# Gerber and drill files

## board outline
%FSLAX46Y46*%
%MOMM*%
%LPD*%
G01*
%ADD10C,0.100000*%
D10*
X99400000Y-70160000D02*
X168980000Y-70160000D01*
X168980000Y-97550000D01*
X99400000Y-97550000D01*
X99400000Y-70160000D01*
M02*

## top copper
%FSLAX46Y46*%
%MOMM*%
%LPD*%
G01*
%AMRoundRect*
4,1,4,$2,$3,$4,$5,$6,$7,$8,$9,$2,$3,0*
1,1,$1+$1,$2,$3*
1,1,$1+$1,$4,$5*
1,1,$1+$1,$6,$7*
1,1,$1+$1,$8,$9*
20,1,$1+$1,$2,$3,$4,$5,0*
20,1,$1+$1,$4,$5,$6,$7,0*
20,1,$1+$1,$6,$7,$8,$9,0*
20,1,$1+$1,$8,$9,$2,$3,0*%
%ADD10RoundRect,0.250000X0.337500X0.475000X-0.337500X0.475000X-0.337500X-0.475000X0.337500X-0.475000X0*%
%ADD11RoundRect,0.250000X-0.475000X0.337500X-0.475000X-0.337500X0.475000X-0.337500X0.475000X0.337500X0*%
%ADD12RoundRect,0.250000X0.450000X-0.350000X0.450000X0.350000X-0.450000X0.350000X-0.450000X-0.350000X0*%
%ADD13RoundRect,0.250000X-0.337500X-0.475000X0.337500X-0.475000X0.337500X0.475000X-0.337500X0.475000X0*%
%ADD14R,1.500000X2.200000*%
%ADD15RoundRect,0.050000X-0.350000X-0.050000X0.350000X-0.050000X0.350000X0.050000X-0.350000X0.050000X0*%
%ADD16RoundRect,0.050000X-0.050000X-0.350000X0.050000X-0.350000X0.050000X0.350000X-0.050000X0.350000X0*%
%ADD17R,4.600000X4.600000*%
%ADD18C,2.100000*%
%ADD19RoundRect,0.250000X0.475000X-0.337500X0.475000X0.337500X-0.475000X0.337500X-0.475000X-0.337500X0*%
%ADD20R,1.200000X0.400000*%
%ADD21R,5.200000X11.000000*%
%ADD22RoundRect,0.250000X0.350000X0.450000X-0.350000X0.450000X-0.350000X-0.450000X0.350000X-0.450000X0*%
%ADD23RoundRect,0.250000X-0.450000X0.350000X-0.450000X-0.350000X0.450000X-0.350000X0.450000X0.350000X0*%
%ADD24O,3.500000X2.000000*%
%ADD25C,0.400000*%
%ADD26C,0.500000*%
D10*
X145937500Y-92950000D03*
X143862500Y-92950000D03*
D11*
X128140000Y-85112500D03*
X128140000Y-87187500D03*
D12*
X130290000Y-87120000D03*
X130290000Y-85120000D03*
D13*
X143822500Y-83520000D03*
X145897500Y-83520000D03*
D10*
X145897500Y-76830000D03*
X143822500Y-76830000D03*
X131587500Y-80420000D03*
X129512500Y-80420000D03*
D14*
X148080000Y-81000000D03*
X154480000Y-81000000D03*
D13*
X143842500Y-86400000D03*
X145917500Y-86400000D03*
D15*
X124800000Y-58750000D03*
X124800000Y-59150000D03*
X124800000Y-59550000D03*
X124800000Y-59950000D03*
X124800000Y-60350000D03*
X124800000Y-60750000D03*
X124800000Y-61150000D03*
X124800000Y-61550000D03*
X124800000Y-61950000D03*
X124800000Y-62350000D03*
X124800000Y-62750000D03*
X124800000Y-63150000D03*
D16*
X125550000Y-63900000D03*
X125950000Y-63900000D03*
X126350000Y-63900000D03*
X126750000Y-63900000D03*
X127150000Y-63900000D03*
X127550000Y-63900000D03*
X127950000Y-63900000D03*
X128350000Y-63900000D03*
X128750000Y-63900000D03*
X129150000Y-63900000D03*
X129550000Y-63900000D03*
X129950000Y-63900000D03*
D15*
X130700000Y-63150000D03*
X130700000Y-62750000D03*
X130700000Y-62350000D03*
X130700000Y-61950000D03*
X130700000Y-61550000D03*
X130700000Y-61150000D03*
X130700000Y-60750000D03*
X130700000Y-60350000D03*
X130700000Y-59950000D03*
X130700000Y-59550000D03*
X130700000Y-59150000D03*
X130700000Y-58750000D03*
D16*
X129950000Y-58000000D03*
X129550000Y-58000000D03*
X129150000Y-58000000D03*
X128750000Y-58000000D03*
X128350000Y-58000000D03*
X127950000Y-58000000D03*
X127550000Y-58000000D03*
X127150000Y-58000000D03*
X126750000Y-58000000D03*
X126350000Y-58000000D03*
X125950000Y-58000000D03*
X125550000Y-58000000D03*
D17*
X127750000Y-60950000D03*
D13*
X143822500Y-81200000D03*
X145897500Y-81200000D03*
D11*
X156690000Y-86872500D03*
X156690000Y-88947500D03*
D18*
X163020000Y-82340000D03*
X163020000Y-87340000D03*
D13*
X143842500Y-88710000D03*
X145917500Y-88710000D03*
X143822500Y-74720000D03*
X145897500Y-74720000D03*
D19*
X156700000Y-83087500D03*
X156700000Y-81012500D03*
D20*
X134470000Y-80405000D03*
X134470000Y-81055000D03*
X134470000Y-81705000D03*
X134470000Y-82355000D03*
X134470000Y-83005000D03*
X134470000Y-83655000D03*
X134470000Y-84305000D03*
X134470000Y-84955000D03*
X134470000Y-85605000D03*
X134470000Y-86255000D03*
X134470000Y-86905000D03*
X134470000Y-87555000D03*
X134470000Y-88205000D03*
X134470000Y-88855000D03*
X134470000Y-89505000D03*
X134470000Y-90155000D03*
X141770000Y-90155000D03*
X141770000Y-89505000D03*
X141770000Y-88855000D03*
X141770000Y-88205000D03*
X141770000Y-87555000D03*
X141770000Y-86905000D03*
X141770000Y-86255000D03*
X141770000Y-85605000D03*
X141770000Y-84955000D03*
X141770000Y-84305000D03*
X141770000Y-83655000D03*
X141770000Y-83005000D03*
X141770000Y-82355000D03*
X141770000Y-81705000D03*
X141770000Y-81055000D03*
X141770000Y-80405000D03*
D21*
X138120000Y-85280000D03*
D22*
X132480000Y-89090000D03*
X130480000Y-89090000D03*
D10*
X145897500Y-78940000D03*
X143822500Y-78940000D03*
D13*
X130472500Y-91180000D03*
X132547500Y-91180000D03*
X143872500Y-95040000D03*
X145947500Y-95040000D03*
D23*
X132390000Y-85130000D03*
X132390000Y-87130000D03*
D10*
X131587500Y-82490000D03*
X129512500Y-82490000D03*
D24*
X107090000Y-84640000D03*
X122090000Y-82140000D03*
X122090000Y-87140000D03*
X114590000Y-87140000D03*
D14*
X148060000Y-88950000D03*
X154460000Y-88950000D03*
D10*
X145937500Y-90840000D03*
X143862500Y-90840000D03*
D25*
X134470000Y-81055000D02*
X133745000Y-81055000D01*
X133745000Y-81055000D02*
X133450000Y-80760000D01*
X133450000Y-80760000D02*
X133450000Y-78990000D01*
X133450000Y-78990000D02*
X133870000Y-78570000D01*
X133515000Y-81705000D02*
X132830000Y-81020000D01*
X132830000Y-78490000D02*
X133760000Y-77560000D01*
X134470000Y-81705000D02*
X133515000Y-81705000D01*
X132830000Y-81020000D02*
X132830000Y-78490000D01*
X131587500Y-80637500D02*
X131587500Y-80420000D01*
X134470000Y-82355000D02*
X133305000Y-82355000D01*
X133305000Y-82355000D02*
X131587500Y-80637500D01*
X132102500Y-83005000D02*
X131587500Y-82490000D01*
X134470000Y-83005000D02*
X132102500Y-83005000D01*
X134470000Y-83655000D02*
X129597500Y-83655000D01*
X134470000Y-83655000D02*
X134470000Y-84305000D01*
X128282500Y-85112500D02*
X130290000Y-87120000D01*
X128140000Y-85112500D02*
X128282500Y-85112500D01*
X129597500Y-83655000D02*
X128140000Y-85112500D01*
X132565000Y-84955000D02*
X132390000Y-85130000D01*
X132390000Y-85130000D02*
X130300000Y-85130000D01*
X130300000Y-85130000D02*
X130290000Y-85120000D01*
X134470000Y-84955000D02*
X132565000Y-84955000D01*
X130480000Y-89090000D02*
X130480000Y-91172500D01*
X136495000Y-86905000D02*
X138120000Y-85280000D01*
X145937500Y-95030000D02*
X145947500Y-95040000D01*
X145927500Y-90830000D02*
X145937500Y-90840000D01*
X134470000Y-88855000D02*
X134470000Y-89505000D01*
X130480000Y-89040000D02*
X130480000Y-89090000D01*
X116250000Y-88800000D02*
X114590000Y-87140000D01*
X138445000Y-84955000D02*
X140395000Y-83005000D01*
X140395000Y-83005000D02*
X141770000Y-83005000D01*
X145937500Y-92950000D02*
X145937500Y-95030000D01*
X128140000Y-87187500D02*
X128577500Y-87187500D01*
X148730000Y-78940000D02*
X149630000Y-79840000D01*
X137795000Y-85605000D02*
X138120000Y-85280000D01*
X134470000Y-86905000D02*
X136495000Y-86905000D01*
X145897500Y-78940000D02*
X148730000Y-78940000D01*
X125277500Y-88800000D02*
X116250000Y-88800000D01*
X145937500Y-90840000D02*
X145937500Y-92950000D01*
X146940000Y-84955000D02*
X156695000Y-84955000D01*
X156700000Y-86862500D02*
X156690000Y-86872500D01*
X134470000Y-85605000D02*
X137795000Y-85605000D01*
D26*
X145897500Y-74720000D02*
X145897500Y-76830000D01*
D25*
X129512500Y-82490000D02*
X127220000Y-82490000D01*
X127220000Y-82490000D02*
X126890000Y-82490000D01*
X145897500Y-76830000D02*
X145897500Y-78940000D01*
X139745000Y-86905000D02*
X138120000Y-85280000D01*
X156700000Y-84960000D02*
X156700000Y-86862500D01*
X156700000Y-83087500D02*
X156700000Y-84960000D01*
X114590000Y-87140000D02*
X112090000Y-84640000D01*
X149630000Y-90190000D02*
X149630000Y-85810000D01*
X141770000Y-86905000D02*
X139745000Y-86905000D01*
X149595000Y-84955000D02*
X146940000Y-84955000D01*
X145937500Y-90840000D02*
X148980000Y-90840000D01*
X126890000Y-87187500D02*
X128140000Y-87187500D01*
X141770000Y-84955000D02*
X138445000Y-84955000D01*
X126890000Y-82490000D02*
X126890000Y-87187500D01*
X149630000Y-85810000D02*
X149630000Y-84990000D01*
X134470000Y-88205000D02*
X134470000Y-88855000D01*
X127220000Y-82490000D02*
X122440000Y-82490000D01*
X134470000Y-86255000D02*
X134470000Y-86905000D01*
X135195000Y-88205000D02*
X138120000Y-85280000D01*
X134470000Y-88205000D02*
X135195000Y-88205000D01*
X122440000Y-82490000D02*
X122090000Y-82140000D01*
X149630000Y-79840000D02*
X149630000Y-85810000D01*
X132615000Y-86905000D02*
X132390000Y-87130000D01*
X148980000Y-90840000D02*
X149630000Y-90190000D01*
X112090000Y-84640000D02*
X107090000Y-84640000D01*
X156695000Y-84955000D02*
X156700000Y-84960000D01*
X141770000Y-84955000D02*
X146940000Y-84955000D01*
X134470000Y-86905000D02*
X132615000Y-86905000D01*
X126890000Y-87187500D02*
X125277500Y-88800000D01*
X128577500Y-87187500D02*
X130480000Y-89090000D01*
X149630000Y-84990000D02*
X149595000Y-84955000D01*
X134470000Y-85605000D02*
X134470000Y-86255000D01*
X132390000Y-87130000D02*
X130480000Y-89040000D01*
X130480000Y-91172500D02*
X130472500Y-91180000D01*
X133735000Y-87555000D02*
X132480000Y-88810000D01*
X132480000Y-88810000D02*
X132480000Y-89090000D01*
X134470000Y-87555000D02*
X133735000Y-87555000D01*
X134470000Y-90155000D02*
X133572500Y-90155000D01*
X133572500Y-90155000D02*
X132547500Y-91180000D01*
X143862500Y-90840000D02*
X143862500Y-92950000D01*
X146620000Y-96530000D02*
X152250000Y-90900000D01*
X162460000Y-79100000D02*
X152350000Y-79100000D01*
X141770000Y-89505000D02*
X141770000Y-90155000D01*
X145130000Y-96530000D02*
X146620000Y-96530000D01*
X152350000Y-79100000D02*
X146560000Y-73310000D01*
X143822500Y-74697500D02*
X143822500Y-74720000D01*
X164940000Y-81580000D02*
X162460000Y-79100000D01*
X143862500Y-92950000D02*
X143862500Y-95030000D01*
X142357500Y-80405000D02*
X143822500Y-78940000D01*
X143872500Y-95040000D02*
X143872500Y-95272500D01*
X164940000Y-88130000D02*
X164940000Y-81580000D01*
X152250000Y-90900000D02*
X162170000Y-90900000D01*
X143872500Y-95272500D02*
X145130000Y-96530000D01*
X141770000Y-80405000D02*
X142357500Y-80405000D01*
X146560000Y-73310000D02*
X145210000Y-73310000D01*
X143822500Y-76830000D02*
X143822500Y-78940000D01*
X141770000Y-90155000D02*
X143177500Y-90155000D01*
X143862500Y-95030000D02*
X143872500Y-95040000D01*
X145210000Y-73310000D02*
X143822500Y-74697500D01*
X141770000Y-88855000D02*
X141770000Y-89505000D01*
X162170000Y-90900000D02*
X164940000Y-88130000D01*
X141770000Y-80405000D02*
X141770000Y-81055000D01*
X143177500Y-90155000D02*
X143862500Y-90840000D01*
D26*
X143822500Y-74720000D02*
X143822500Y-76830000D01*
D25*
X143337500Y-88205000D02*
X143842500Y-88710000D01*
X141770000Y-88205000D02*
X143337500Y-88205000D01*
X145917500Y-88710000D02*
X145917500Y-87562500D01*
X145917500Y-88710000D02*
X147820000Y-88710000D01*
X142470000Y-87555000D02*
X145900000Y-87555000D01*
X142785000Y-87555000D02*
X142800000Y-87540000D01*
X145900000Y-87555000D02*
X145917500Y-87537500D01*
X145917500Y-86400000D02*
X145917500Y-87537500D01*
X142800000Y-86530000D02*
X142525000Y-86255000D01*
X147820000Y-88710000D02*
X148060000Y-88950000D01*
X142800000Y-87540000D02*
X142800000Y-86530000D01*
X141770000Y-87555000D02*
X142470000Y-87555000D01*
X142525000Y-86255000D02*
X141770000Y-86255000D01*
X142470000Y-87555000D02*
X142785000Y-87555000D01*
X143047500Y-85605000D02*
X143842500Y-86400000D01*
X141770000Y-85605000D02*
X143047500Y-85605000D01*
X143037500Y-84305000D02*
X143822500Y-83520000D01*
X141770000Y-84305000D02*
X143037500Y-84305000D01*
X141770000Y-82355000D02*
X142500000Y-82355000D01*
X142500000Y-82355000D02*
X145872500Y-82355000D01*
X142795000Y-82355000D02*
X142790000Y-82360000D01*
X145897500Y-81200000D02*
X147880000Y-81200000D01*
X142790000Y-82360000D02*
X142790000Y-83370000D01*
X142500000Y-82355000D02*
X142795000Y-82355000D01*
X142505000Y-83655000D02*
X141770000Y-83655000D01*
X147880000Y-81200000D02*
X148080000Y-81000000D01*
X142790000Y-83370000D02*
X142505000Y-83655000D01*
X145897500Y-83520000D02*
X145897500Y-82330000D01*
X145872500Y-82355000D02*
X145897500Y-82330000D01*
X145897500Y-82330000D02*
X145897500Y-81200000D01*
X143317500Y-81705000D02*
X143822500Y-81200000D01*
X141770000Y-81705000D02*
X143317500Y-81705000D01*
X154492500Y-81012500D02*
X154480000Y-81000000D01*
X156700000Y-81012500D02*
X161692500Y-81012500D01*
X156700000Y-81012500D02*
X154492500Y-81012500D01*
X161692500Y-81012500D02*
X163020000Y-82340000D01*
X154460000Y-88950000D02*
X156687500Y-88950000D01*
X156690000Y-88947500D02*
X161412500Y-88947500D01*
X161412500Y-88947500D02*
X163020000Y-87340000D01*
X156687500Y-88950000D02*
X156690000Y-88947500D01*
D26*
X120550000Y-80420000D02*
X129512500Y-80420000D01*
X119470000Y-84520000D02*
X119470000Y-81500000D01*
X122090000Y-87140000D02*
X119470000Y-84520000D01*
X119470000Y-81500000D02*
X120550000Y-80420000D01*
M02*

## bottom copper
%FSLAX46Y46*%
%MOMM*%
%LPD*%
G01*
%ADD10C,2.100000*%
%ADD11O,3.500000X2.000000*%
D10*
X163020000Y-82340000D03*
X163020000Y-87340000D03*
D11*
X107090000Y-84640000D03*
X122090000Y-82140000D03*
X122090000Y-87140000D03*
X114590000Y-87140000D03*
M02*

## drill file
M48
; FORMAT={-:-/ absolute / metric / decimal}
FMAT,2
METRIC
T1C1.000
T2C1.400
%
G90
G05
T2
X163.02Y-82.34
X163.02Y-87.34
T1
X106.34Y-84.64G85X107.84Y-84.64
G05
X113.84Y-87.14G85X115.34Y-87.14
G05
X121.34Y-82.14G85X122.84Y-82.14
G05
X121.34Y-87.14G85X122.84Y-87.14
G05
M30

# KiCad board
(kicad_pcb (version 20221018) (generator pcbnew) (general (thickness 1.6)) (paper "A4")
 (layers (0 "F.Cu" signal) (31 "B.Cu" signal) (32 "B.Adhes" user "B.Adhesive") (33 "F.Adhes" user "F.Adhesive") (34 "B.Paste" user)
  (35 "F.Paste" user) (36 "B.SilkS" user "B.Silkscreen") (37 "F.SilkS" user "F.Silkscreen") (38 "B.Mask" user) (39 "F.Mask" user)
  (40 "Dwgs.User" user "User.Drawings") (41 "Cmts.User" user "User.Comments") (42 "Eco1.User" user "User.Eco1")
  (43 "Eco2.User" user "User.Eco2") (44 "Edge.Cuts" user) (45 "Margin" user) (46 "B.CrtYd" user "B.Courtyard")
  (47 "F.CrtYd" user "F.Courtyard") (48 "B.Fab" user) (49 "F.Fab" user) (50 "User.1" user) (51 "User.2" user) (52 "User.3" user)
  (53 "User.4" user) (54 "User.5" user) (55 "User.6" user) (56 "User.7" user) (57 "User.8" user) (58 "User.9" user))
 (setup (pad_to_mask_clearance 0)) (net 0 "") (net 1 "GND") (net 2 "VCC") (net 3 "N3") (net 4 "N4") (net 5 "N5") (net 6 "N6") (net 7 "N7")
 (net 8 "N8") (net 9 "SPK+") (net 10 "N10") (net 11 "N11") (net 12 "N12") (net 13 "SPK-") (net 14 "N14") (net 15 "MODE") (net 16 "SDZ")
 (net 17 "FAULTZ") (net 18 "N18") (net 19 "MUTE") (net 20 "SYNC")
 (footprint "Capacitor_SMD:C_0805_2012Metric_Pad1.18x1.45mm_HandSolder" (layer "F.Cu") (at 144.9 92.95 180)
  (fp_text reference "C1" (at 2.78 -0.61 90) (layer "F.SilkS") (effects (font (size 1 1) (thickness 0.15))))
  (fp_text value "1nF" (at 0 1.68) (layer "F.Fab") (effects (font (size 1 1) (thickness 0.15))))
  (pad "1" smd roundrect (at -1.0375 0 180) (size 1.175 1.45) (layers "F.Cu" "F.Paste" "F.Mask") (roundrect_rratio 0.212766) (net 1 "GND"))
  (pad "2" smd roundrect (at 1.0375 0 180) (size 1.175 1.45) (layers "F.Cu" "F.Paste" "F.Mask") (roundrect_rratio 0.212766) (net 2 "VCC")))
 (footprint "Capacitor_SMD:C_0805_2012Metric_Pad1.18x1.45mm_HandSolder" (layer "F.Cu") (at 128.14 86.15 -90)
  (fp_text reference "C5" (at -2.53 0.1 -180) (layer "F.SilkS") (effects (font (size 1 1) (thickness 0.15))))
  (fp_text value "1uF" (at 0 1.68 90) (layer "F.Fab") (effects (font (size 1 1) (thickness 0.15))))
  (pad "1" smd roundrect (at -1.0375 0 270) (size 1.175 1.45) (layers "F.Cu" "F.Paste" "F.Mask") (roundrect_rratio 0.212766) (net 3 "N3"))
  (pad "2" smd roundrect (at 1.0375 0 270) (size 1.175 1.45) (layers "F.Cu" "F.Paste" "F.Mask") (roundrect_rratio 0.212766) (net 1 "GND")))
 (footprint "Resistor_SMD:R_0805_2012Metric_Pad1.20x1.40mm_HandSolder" (layer "F.Cu") (at 130.29 86.12 90)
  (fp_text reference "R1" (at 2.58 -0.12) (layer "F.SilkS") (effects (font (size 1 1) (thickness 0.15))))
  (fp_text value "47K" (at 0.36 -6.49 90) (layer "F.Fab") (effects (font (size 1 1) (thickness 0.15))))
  (pad "1" smd roundrect (at -1 0 90) (size 1.2 1.4) (layers "F.Cu" "F.Paste" "F.Mask") (roundrect_rratio 0.208333) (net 3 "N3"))
  (pad "2" smd roundrect (at 1 0 90) (size 1.2 1.4) (layers "F.Cu" "F.Paste" "F.Mask") (roundrect_rratio 0.208333) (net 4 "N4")))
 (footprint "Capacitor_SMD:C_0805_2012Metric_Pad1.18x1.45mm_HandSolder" (layer "F.Cu") (at 144.86 83.52)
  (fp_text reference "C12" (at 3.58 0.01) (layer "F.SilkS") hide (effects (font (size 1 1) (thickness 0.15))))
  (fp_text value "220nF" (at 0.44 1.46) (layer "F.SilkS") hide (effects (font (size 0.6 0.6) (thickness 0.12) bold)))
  (pad "1" smd roundrect (at -1.0375 0) (size 1.175 1.45) (layers "F.Cu" "F.Paste" "F.Mask") (roundrect_rratio 0.212766) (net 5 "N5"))
  (pad "2" smd roundrect (at 1.0375 0) (size 1.175 1.45) (layers "F.Cu" "F.Paste" "F.Mask") (roundrect_rratio 0.212766) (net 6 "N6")))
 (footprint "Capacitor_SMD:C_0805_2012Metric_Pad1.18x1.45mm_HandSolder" (layer "F.Cu") (at 144.86 76.83 180)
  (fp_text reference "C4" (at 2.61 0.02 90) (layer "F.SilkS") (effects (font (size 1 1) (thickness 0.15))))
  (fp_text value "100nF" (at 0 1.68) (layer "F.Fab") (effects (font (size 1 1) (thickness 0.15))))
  (pad "1" smd roundrect (at -1.0375 0 180) (size 1.175 1.45) (layers "F.Cu" "F.Paste" "F.Mask") (roundrect_rratio 0.212766) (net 1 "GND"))
  (pad "2" smd roundrect (at 1.0375 0 180) (size 1.175 1.45) (layers "F.Cu" "F.Paste" "F.Mask") (roundrect_rratio 0.212766) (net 2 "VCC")))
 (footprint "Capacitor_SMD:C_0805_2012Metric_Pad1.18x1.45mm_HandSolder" (layer "F.Cu") (at 130.55 80.42 180)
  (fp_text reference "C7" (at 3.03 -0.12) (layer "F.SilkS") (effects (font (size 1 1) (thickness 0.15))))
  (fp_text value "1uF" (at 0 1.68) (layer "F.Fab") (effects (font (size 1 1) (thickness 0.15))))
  (pad "1" smd roundrect (at -1.0375 0 180) (size 1.175 1.45) (layers "F.Cu" "F.Paste" "F.Mask") (roundrect_rratio 0.212766) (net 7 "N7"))
  (pad "2" smd roundrect (at 1.0375 0 180) (size 1.175 1.45) (layers "F.Cu" "F.Paste" "F.Mask") (roundrect_rratio 0.212766) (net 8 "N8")))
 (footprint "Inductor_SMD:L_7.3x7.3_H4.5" (layer "F.Cu") (at 151.28 81)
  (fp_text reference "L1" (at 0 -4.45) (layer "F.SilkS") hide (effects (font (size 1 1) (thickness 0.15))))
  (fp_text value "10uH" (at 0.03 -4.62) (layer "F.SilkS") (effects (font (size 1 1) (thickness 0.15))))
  (pad "1" smd rect (at -3.2 0) (size 1.5 2.2) (layers "F.Cu" "F.Paste" "F.Mask") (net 6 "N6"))
  (pad "2" smd rect (at 3.2 0) (size 1.5 2.2) (layers "F.Cu" "F.Paste" "F.Mask") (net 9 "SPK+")))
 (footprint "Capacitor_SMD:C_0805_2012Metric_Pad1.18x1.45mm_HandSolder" (layer "F.Cu") (at 144.88 86.4)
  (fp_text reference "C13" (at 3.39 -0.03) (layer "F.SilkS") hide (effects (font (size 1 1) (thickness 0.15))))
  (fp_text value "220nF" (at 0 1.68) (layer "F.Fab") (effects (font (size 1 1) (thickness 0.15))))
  (pad "1" smd roundrect (at -1.0375 0) (size 1.175 1.45) (layers "F.Cu" "F.Paste" "F.Mask") (roundrect_rratio 0.212766) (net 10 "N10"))
  (pad "2" smd roundrect (at 1.0375 0) (size 1.175 1.45) (layers "F.Cu" "F.Paste" "F.Mask") (roundrect_rratio 0.212766) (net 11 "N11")))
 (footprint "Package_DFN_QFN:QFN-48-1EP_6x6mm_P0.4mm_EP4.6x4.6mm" (layer "F.Cu") (at 127.75 60.95)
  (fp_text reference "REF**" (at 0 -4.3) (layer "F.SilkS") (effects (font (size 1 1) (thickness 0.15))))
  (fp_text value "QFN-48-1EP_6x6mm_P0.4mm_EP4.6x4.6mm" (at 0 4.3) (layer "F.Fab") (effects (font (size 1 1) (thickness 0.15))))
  (pad "" smd roundrect (at -1.53 -1.53) (size 1.24 1.24) (layers "F.Paste") (roundrect_rratio 0.201613))
  (pad "" smd roundrect (at -1.53 0) (size 1.24 1.24) (layers "F.Paste") (roundrect_rratio 0.201613))
  (pad "" smd roundrect (at -1.53 1.53) (size 1.24 1.24) (layers "F.Paste") (roundrect_rratio 0.201613))
  (pad "" smd roundrect (at 0 -1.53) (size 1.24 1.24) (layers "F.Paste") (roundrect_rratio 0.201613))
  (pad "" smd roundrect (at 0 0) (size 1.24 1.24) (layers "F.Paste") (roundrect_rratio 0.201613))
  (pad "" smd roundrect (at 0 1.53) (size 1.24 1.24) (layers "F.Paste") (roundrect_rratio 0.201613))
  (pad "" smd roundrect (at 1.53 -1.53) (size 1.24 1.24) (layers "F.Paste") (roundrect_rratio 0.201613))
  (pad "" smd roundrect (at 1.53 0) (size 1.24 1.24) (layers "F.Paste") (roundrect_rratio 0.201613))
  (pad "" smd roundrect (at 1.53 1.53) (size 1.24 1.24) (layers "F.Paste") (roundrect_rratio 0.201613))
  (pad "1" smd roundrect (at -2.95 -2.2) (size 0.8 0.2) (layers "F.Cu" "F.Paste" "F.Mask") (roundrect_rratio 0.25))
  (pad "2" smd roundrect (at -2.95 -1.8) (size 0.8 0.2) (layers "F.Cu" "F.Paste" "F.Mask") (roundrect_rratio 0.25))
  (pad "3" smd roundrect (at -2.95 -1.4) (size 0.8 0.2) (layers "F.Cu" "F.Paste" "F.Mask") (roundrect_rratio 0.25))
  (pad "4" smd roundrect (at -2.95 -1) (size 0.8 0.2) (layers "F.Cu" "F.Paste" "F.Mask") (roundrect_rratio 0.25))
  (pad "5" smd roundrect (at -2.95 -0.6) (size 0.8 0.2) (layers "F.Cu" "F.Paste" "F.Mask") (roundrect_rratio 0.25))
  (pad "6" smd roundrect (at -2.95 -0.2) (size 0.8 0.2) (layers "F.Cu" "F.Paste" "F.Mask") (roundrect_rratio 0.25))
  (pad "7" smd roundrect (at -2.95 0.2) (size 0.8 0.2) (layers "F.Cu" "F.Paste" "F.Mask") (roundrect_rratio 0.25))
  (pad "8" smd roundrect (at -2.95 0.6) (size 0.8 0.2) (layers "F.Cu" "F.Paste" "F.Mask") (roundrect_rratio 0.25))
  (pad "9" smd roundrect (at -2.95 1) (size 0.8 0.2) (layers "F.Cu" "F.Paste" "F.Mask") (roundrect_rratio 0.25))
  (pad "10" smd roundrect (at -2.95 1.4) (size 0.8 0.2) (layers "F.Cu" "F.Paste" "F.Mask") (roundrect_rratio 0.25))
  (pad "11" smd roundrect (at -2.95 1.8) (size 0.8 0.2) (layers "F.Cu" "F.Paste" "F.Mask") (roundrect_rratio 0.25))
  (pad "12" smd roundrect (at -2.95 2.2) (size 0.8 0.2) (layers "F.Cu" "F.Paste" "F.Mask") (roundrect_rratio 0.25))
  (pad "13" smd roundrect (at -2.2 2.95) (size 0.2 0.8) (layers "F.Cu" "F.Paste" "F.Mask") (roundrect_rratio 0.25))
  (pad "14" smd roundrect (at -1.8 2.95) (size 0.2 0.8) (layers "F.Cu" "F.Paste" "F.Mask") (roundrect_rratio 0.25))
  (pad "15" smd roundrect (at -1.4 2.95) (size 0.2 0.8) (layers "F.Cu" "F.Paste" "F.Mask") (roundrect_rratio 0.25))
  (pad "16" smd roundrect (at -1 2.95) (size 0.2 0.8) (layers "F.Cu" "F.Paste" "F.Mask") (roundrect_rratio 0.25))
  (pad "17" smd roundrect (at -0.6 2.95) (size 0.2 0.8) (layers "F.Cu" "F.Paste" "F.Mask") (roundrect_rratio 0.25))
  (pad "18" smd roundrect (at -0.2 2.95) (size 0.2 0.8) (layers "F.Cu" "F.Paste" "F.Mask") (roundrect_rratio 0.25))
  (pad "19" smd roundrect (at 0.2 2.95) (size 0.2 0.8) (layers "F.Cu" "F.Paste" "F.Mask") (roundrect_rratio 0.25))
  (pad "20" smd roundrect (at 0.6 2.95) (size 0.2 0.8) (layers "F.Cu" "F.Paste" "F.Mask") (roundrect_rratio 0.25))
  (pad "21" smd roundrect (at 1 2.95) (size 0.2 0.8) (layers "F.Cu" "F.Paste" "F.Mask") (roundrect_rratio 0.25))
  (pad "22" smd roundrect (at 1.4 2.95) (size 0.2 0.8) (layers "F.Cu" "F.Paste" "F.Mask") (roundrect_rratio 0.25))
  (pad "23" smd roundrect (at 1.8 2.95) (size 0.2 0.8) (layers "F.Cu" "F.Paste" "F.Mask") (roundrect_rratio 0.25))
  (pad "24" smd roundrect (at 2.2 2.95) (size 0.2 0.8) (layers "F.Cu" "F.Paste" "F.Mask") (roundrect_rratio 0.25))
  (pad "25" smd roundrect (at 2.95 2.2) (size 0.8 0.2) (layers "F.Cu" "F.Paste" "F.Mask") (roundrect_rratio 0.25))
  (pad "26" smd roundrect (at 2.95 1.8) (size 0.8 0.2) (layers "F.Cu" "F.Paste" "F.Mask") (roundrect_rratio 0.25))
  (pad "27" smd roundrect (at 2.95 1.4) (size 0.8 0.2) (layers "F.Cu" "F.Paste" "F.Mask") (roundrect_rratio 0.25))
  (pad "28" smd roundrect (at 2.95 1) (size 0.8 0.2) (layers "F.Cu" "F.Paste" "F.Mask") (roundrect_rratio 0.25))
  (pad "29" smd roundrect (at 2.95 0.6) (size 0.8 0.2) (layers "F.Cu" "F.Paste" "F.Mask") (roundrect_rratio 0.25))
  (pad "30" smd roundrect (at 2.95 0.2) (size 0.8 0.2) (layers "F.Cu" "F.Paste" "F.Mask") (roundrect_rratio 0.25))
  (pad "31" smd roundrect (at 2.95 -0.2) (size 0.8 0.2) (layers "F.Cu" "F.Paste" "F.Mask") (roundrect_rratio 0.25))
  (pad "32" smd roundrect (at 2.95 -0.6) (size 0.8 0.2) (layers "F.Cu" "F.Paste" "F.Mask") (roundrect_rratio 0.25))
  (pad "33" smd roundrect (at 2.95 -1) (size 0.8 0.2) (layers "F.Cu" "F.Paste" "F.Mask") (roundrect_rratio 0.25))
  (pad "34" smd roundrect (at 2.95 -1.4) (size 0.8 0.2) (layers "F.Cu" "F.Paste" "F.Mask") (roundrect_rratio 0.25))
  (pad "35" smd roundrect (at 2.95 -1.8) (size 0.8 0.2) (layers "F.Cu" "F.Paste" "F.Mask") (roundrect_rratio 0.25))
  (pad "36" smd roundrect (at 2.95 -2.2) (size 0.8 0.2) (layers "F.Cu" "F.Paste" "F.Mask") (roundrect_rratio 0.25))
  (pad "37" smd roundrect (at 2.2 -2.95) (size 0.2 0.8) (layers "F.Cu" "F.Paste" "F.Mask") (roundrect_rratio 0.25))
  (pad "38" smd roundrect (at 1.8 -2.95) (size 0.2 0.8) (layers "F.Cu" "F.Paste" "F.Mask") (roundrect_rratio 0.25))
  (pad "39" smd roundrect (at 1.4 -2.95) (size 0.2 0.8) (layers "F.Cu" "F.Paste" "F.Mask") (roundrect_rratio 0.25))
  (pad "40" smd roundrect (at 1 -2.95) (size 0.2 0.8) (layers "F.Cu" "F.Paste" "F.Mask") (roundrect_rratio 0.25))
  (pad "41" smd roundrect (at 0.6 -2.95) (size 0.2 0.8) (layers "F.Cu" "F.Paste" "F.Mask") (roundrect_rratio 0.25))
  (pad "42" smd roundrect (at 0.2 -2.95) (size 0.2 0.8) (layers "F.Cu" "F.Paste" "F.Mask") (roundrect_rratio 0.25))
  (pad "43" smd roundrect (at -0.2 -2.95) (size 0.2 0.8) (layers "F.Cu" "F.Paste" "F.Mask") (roundrect_rratio 0.25))
  (pad "44" smd roundrect (at -0.6 -2.95) (size 0.2 0.8) (layers "F.Cu" "F.Paste" "F.Mask") (roundrect_rratio 0.25))
  (pad "45" smd roundrect (at -1 -2.95) (size 0.2 0.8) (layers "F.Cu" "F.Paste" "F.Mask") (roundrect_rratio 0.25))
  (pad "46" smd roundrect (at -1.4 -2.95) (size 0.2 0.8) (layers "F.Cu" "F.Paste" "F.Mask") (roundrect_rratio 0.25))
  (pad "47" smd roundrect (at -1.8 -2.95) (size 0.2 0.8) (layers "F.Cu" "F.Paste" "F.Mask") (roundrect_rratio 0.25))
  (pad "48" smd roundrect (at -2.2 -2.95) (size 0.2 0.8) (layers "F.Cu" "F.Paste" "F.Mask") (roundrect_rratio 0.25))
  (pad "49" smd rect (at 0 0) (size 4.6 4.6) (layers "F.Cu" "F.Mask")))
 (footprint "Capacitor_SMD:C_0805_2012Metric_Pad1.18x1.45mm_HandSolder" (layer "F.Cu") (at 144.86 81.2)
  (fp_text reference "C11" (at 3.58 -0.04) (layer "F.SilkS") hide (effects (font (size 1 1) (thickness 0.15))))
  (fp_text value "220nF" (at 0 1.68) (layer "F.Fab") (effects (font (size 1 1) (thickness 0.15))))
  (pad "1" smd roundrect (at -1.0375 0) (size 1.175 1.45) (layers "F.Cu" "F.Paste" "F.Mask") (roundrect_rratio 0.212766) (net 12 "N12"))
  (pad "2" smd roundrect (at 1.0375 0) (size 1.175 1.45) (layers "F.Cu" "F.Paste" "F.Mask") (roundrect_rratio 0.212766) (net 6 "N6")))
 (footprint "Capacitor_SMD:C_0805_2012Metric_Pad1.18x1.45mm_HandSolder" (layer "F.Cu") (at 156.69 87.91 -90)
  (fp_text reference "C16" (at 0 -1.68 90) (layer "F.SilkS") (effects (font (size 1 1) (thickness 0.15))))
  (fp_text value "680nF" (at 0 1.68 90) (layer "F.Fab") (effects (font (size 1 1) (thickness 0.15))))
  (pad "1" smd roundrect (at -1.0375 0 270) (size 1.175 1.45) (layers "F.Cu" "F.Paste" "F.Mask") (roundrect_rratio 0.212766) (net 1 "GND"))
  (pad "2" smd roundrect (at 1.0375 0 270) (size 1.175 1.45) (layers "F.Cu" "F.Paste" "F.Mask") (roundrect_rratio 0.212766) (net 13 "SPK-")))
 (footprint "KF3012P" (layer "F.Cu") (at 163.02 82.34 -90)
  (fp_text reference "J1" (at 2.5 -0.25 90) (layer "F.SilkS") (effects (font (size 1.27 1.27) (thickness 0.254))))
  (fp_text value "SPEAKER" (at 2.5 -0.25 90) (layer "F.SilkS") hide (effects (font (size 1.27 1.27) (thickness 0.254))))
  (pad "1" thru_hole circle (at 0 0 270) (size 2.1 2.1) (drill 1.4) (layers "*.Cu" "*.Mask") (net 9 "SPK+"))
  (pad "2" thru_hole circle (at 5 0 270) (size 2.1 2.1) (drill 1.4) (layers "*.Cu" "*.Mask") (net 13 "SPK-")))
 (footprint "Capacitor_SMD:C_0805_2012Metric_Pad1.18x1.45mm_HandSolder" (layer "F.Cu") (at 144.88 88.71)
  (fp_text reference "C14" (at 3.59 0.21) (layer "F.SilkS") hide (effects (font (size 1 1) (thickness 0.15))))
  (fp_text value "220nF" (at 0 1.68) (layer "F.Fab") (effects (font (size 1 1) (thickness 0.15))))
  (pad "1" smd roundrect (at -1.0375 0) (size 1.175 1.45) (layers "F.Cu" "F.Paste" "F.Mask") (roundrect_rratio 0.212766) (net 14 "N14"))
  (pad "2" smd roundrect (at 1.0375 0) (size 1.175 1.45) (layers "F.Cu" "F.Paste" "F.Mask") (roundrect_rratio 0.212766) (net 11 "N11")))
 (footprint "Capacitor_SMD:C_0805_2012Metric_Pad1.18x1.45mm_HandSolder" (layer "F.Cu") (at 144.86 74.72)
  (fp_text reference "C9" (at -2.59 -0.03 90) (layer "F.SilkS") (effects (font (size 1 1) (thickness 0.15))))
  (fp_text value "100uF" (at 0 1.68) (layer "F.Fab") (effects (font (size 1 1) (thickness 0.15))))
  (pad "1" smd roundrect (at -1.0375 0) (size 1.175 1.45) (layers "F.Cu" "F.Paste" "F.Mask") (roundrect_rratio 0.212766) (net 2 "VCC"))
  (pad "2" smd roundrect (at 1.0375 0) (size 1.175 1.45) (layers "F.Cu" "F.Paste" "F.Mask") (roundrect_rratio 0.212766) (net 1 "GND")))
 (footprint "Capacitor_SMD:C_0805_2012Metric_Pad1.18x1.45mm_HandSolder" (layer "F.Cu") (at 156.7 82.05 90)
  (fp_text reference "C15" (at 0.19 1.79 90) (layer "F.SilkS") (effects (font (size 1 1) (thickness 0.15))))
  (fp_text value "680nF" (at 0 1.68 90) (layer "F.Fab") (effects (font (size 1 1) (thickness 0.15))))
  (pad "1" smd roundrect (at -1.0375 0 90) (size 1.175 1.45) (layers "F.Cu" "F.Paste" "F.Mask") (roundrect_rratio 0.212766) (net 1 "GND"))
  (pad "2" smd roundrect (at 1.0375 0 90) (size 1.175 1.45) (layers "F.Cu" "F.Paste" "F.Mask") (roundrect_rratio 0.212766) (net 9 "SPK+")))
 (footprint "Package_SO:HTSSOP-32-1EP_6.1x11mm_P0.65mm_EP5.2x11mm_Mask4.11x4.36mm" (layer "F.Cu") (at 138.12 85.28)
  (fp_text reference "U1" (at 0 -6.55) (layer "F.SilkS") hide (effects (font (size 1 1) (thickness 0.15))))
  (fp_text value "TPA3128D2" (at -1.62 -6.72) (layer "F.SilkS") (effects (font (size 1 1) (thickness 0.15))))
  (pad "" smd rect (at -1.37 -1.46) (size 1.07 1.16) (layers "F.Paste"))
  (pad "" smd rect (at -1.37 0) (size 1.07 1.16) (layers "F.Paste"))
  (pad "" smd rect (at -1.37 1.46) (size 1.07 1.16) (layers "F.Paste"))
  (pad "" smd rect (at 0 -1.46) (size 1.07 1.16) (layers "F.Paste"))
  (pad "" smd rect (at 0 0) (size 1.07 1.16) (layers "F.Paste"))
  (pad "" smd rect (at 0 0) (size 4.11 4.36) (layers "F.Mask"))
  (pad "" smd rect (at 0 1.46) (size 1.07 1.16) (layers "F.Paste"))
  (pad "" smd rect (at 1.37 -1.46) (size 1.07 1.16) (layers "F.Paste"))
  (pad "" smd rect (at 1.37 0) (size 1.07 1.16) (layers "F.Paste"))
  (pad "" smd rect (at 1.37 1.46) (size 1.07 1.16) (layers "F.Paste"))
  (pad "1" smd rect (at -3.65 -4.875) (size 1.2 0.4) (layers "F.Cu" "F.Paste" "F.Mask") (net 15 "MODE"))
  (pad "2" smd rect (at -3.65 -4.225) (size 1.2 0.4) (layers "F.Cu" "F.Paste" "F.Mask") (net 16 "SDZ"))
  (pad "3" smd rect (at -3.65 -3.575) (size 1.2 0.4) (layers "F.Cu" "F.Paste" "F.Mask") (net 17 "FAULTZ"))
  (pad "4" smd rect (at -3.65 -2.925) (size 1.2 0.4) (layers "F.Cu" "F.Paste" "F.Mask") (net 7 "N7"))
  (pad "5" smd rect (at -3.65 -2.275) (size 1.2 0.4) (layers "F.Cu" "F.Paste" "F.Mask") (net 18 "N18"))
  (pad "6" smd rect (at -3.65 -1.625) (size 1.2 0.4) (layers "F.Cu" "F.Paste" "F.Mask") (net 3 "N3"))
  (pad "7" smd rect (at -3.65 -0.975) (size 1.2 0.4) (layers "F.Cu" "F.Paste" "F.Mask") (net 3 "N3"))
  (pad "8" smd rect (at -3.65 -0.325) (size 1.2 0.4) (layers "F.Cu" "F.Paste" "F.Mask") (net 4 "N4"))
  (pad "9" smd rect (at -3.65 0.325) (size 1.2 0.4) (layers "F.Cu" "F.Paste" "F.Mask") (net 1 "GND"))
  (pad "10" smd rect (at -3.65 0.975) (size 1.2 0.4) (layers "F.Cu" "F.Paste" "F.Mask") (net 1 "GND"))
  (pad "11" smd rect (at -3.65 1.625) (size 1.2 0.4) (layers "F.Cu" "F.Paste" "F.Mask") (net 1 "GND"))
  (pad "12" smd rect (at -3.65 2.275) (size 1.2 0.4) (layers "F.Cu" "F.Paste" "F.Mask") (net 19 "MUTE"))
  (pad "13" smd rect (at -3.65 2.925) (size 1.2 0.4) (layers "F.Cu" "F.Paste" "F.Mask") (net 1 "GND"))
  (pad "14" smd rect (at -3.65 3.575) (size 1.2 0.4) (layers "F.Cu" "F.Paste" "F.Mask") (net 1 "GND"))
  (pad "15" smd rect (at -3.65 4.225) (size 1.2 0.4) (layers "F.Cu" "F.Paste" "F.Mask") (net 1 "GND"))
  (pad "16" smd rect (at -3.65 4.875) (size 1.2 0.4) (layers "F.Cu" "F.Paste" "F.Mask") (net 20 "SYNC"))
  (pad "17" smd rect (at 3.65 4.875) (size 1.2 0.4) (layers "F.Cu" "F.Paste" "F.Mask") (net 2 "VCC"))
  (pad "18" smd rect (at 3.65 4.225) (size 1.2 0.4) (layers "F.Cu" "F.Paste" "F.Mask") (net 2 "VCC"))
  (pad "19" smd rect (at 3.65 3.575) (size 1.2 0.4) (layers "F.Cu" "F.Paste" "F.Mask") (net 2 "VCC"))
  (pad "20" smd rect (at 3.65 2.925) (size 1.2 0.4) (layers "F.Cu" "F.Paste" "F.Mask") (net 14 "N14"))
  (pad "21" smd rect (at 3.65 2.275) (size 1.2 0.4) (layers "F.Cu" "F.Paste" "F.Mask") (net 11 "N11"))
  (pad "22" smd rect (at 3.65 1.625) (size 1.2 0.4) (layers "F.Cu" "F.Paste" "F.Mask") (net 1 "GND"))
  (pad "23" smd rect (at 3.65 0.975) (size 1.2 0.4) (layers "F.Cu" "F.Paste" "F.Mask") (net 11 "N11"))
  (pad "24" smd rect (at 3.65 0.325) (size 1.2 0.4) (layers "F.Cu" "F.Paste" "F.Mask") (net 10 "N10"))
  (pad "25" smd rect (at 3.65 -0.325) (size 1.2 0.4) (layers "F.Cu" "F.Paste" "F.Mask") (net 1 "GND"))
  (pad "26" smd rect (at 3.65 -0.975) (size 1.2 0.4) (layers "F.Cu" "F.Paste" "F.Mask") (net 5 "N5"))
  (pad "27" smd rect (at 3.65 -1.625) (size 1.2 0.4) (layers "F.Cu" "F.Paste" "F.Mask") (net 6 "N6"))
  (pad "28" smd rect (at 3.65 -2.275) (size 1.2 0.4) (layers "F.Cu" "F.Paste" "F.Mask") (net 1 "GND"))
  (pad "29" smd rect (at 3.65 -2.925) (size 1.2 0.4) (layers "F.Cu" "F.Paste" "F.Mask") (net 6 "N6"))
  (pad "30" smd rect (at 3.65 -3.575) (size 1.2 0.4) (layers "F.Cu" "F.Paste" "F.Mask") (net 12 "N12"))
  (pad "31" smd rect (at 3.65 -4.225) (size 1.2 0.4) (layers "F.Cu" "F.Paste" "F.Mask") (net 2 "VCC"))
  (pad "32" smd rect (at 3.65 -4.875) (size 1.2 0.4) (layers "F.Cu" "F.Paste" "F.Mask") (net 2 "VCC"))
  (pad "33" smd rect (at 0 0) (size 5.2 11) (layers "F.Cu")))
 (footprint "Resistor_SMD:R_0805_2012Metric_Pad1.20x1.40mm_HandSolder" (layer "F.Cu") (at 131.48 89.09 180)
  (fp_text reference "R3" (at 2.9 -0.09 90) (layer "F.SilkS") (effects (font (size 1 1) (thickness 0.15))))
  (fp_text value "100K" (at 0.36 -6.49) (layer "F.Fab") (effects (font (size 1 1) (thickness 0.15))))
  (pad "1" smd roundrect (at -1 0 180) (size 1.2 1.4) (layers "F.Cu" "F.Paste" "F.Mask") (roundrect_rratio 0.208333) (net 19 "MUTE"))
  (pad "2" smd roundrect (at 1 0 180) (size 1.2 1.4) (layers "F.Cu" "F.Paste" "F.Mask") (roundrect_rratio 0.208333) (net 1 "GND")))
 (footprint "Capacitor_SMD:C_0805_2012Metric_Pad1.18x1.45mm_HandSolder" (layer "F.Cu") (at 144.86 78.94 180)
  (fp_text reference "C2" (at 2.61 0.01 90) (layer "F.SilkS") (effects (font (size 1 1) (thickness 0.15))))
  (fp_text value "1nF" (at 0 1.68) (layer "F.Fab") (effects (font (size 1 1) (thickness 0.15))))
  (pad "1" smd roundrect (at -1.0375 0 180) (size 1.175 1.45) (layers "F.Cu" "F.Paste" "F.Mask") (roundrect_rratio 0.212766) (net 1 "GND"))
  (pad "2" smd roundrect (at 1.0375 0 180) (size 1.175 1.45) (layers "F.Cu" "F.Paste" "F.Mask") (roundrect_rratio 0.212766) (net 2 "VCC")))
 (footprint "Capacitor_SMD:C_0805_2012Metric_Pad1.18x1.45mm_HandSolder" (layer "F.Cu") (at 131.51 91.18)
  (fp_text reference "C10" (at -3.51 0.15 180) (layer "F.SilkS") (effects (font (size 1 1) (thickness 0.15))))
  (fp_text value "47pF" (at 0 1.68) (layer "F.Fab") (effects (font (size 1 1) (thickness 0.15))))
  (pad "1" smd roundrect (at -1.0375 0) (size 1.175 1.45) (layers "F.Cu" "F.Paste" "F.Mask") (roundrect_rratio 0.212766) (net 1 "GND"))
  (pad "2" smd roundrect (at 1.0375 0) (size 1.175 1.45) (layers "F.Cu" "F.Paste" "F.Mask") (roundrect_rratio 0.212766) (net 20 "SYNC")))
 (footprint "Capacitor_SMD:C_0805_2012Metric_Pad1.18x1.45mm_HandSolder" (layer "F.Cu") (at 144.91 95.04)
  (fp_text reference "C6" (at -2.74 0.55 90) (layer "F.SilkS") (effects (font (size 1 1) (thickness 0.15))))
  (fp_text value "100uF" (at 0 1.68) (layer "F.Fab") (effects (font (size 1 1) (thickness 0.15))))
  (pad "1" smd roundrect (at -1.0375 0) (size 1.175 1.45) (layers "F.Cu" "F.Paste" "F.Mask") (roundrect_rratio 0.212766) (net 2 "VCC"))
  (pad "2" smd roundrect (at 1.0375 0) (size 1.175 1.45) (layers "F.Cu" "F.Paste" "F.Mask") (roundrect_rratio 0.212766) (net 1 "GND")))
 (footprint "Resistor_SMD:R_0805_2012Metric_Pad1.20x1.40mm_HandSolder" (layer "F.Cu") (at 132.39 86.13 -90)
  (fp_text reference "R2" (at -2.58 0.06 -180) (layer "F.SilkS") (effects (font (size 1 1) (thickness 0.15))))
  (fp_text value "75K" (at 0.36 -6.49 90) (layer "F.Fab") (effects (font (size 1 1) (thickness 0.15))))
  (pad "1" smd roundrect (at -1 0 270) (size 1.2 1.4) (layers "F.Cu" "F.Paste" "F.Mask") (roundrect_rratio 0.208333) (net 4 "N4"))
  (pad "2" smd roundrect (at 1 0 270) (size 1.2 1.4) (layers "F.Cu" "F.Paste" "F.Mask") (roundrect_rratio 0.208333) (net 1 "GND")))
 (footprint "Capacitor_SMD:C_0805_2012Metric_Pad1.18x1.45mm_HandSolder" (layer "F.Cu") (at 130.55 82.49 180)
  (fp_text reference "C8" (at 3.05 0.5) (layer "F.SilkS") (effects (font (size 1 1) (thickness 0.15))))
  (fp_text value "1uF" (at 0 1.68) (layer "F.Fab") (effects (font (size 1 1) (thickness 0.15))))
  (pad "1" smd roundrect (at -1.0375 0 180) (size 1.175 1.45) (layers "F.Cu" "F.Paste" "F.Mask") (roundrect_rratio 0.212766) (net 18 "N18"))
  (pad "2" smd roundrect (at 1.0375 0 180) (size 1.175 1.45) (layers "F.Cu" "F.Paste" "F.Mask") (roundrect_rratio 0.212766) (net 1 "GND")))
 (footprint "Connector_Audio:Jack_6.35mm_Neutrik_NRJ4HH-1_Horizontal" (layer "F.Cu") (at 118.09 90.14 180)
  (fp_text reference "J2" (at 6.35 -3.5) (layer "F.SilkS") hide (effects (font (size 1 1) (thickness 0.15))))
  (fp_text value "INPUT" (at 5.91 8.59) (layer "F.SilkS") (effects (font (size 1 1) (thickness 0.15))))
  (pad "G" thru_hole oval (at 11 5.5) (size 3.5 2) (drill oval 2.5 1) (layers "*.Cu" "*.Mask") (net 1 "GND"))
  (pad "R" thru_hole oval (at -4 8) (size 3.5 2) (drill oval 2.5 1) (layers "*.Cu" "*.Mask") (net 1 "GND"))
  (pad "S" thru_hole oval (at -4 3) (size 3.5 2) (drill oval 2.5 1) (layers "*.Cu" "*.Mask") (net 8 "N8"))
  (pad "T" thru_hole oval (at 3.5 3) (size 3.5 2) (drill oval 2.5 1) (layers "*.Cu" "*.Mask") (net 1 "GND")))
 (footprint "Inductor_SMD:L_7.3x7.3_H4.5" (layer "F.Cu") (at 151.26 88.95)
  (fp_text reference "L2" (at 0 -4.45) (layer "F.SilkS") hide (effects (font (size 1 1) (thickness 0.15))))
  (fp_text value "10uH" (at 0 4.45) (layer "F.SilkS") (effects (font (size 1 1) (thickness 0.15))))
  (pad "1" smd rect (at -3.2 0) (size 1.5 2.2) (layers "F.Cu" "F.Paste" "F.Mask") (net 11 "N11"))
  (pad "2" smd rect (at 3.2 0) (size 1.5 2.2) (layers "F.Cu" "F.Paste" "F.Mask") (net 13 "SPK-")))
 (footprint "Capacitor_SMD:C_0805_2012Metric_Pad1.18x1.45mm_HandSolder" (layer "F.Cu") (at 144.9 90.84 180)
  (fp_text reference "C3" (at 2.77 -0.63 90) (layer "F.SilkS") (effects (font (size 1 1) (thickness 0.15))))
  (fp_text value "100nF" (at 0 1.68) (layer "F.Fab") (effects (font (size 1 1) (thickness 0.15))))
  (pad "1" smd roundrect (at -1.0375 0 180) (size 1.175 1.45) (layers "F.Cu" "F.Paste" "F.Mask") (roundrect_rratio 0.212766) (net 1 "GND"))
  (pad "2" smd roundrect (at 1.0375 0 180) (size 1.175 1.45) (layers "F.Cu" "F.Paste" "F.Mask") (roundrect_rratio 0.212766) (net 2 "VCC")))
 (gr_rect (start 99.4 70.16) (end 168.98 97.55) (stroke (width 0.1) (type default)) (fill none) (layer "Edge.Cuts"))
 (segment (start 134.47 81.055) (end 133.745 81.055) (width 0.4) (layer "F.Cu") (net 16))
 (segment (start 133.745 81.055) (end 133.45 80.76) (width 0.4) (layer "F.Cu") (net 16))
 (segment (start 133.45 80.76) (end 133.45 78.99) (width 0.4) (layer "F.Cu") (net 16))
 (segment (start 133.45 78.99) (end 133.87 78.57) (width 0.4) (layer "F.Cu") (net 16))
 (segment (start 133.515 81.705) (end 132.83 81.02) (width 0.4) (layer "F.Cu") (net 17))
 (segment (start 132.83 78.49) (end 133.76 77.56) (width 0.4) (layer "F.Cu") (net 17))
 (segment (start 134.47 81.705) (end 133.515 81.705) (width 0.4) (layer "F.Cu") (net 17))
 (segment (start 132.83 81.02) (end 132.83 78.49) (width 0.4) (layer "F.Cu") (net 17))
 (segment (start 131.5875 80.6375) (end 131.5875 80.42) (width 0.4) (layer "F.Cu") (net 7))
 (segment (start 134.47 82.355) (end 133.305 82.355) (width 0.4) (layer "F.Cu") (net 7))
 (segment (start 133.305 82.355) (end 131.5875 80.6375) (width 0.4) (layer "F.Cu") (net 7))
 (segment (start 132.1025 83.005) (end 131.5875 82.49) (width 0.4) (layer "F.Cu") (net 18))
 (segment (start 134.47 83.005) (end 132.1025 83.005) (width 0.4) (layer "F.Cu") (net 18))
 (segment (start 134.47 83.655) (end 129.5975 83.655) (width 0.4) (layer "F.Cu") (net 3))
 (segment (start 134.47 83.655) (end 134.47 84.305) (width 0.4) (layer "F.Cu") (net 3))
 (segment (start 128.2825 85.1125) (end 130.29 87.12) (width 0.4) (layer "F.Cu") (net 3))
 (segment (start 128.14 85.1125) (end 128.2825 85.1125) (width 0.4) (layer "F.Cu") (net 3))
 (segment (start 129.5975 83.655) (end 128.14 85.1125) (width 0.4) (layer "F.Cu") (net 3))
 (segment (start 132.565 84.955) (end 132.39 85.13) (width 0.4) (layer "F.Cu") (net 4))
 (segment (start 132.39 85.13) (end 130.3 85.13) (width 0.4) (layer "F.Cu") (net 4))
 (segment (start 130.3 85.13) (end 130.29 85.12) (width 0.4) (layer "F.Cu") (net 4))
 (segment (start 134.47 84.955) (end 132.565 84.955) (width 0.4) (layer "F.Cu") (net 4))
 (segment (start 130.48 89.09) (end 130.48 91.1725) (width 0.4) (layer "F.Cu") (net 1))
 (segment (start 136.495 86.905) (end 138.12 85.28) (width 0.4) (layer "F.Cu") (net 1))
 (segment (start 145.9375 95.03) (end 145.9475 95.04) (width 0.4) (layer "F.Cu") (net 1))
 (segment (start 145.9275 90.83) (end 145.9375 90.84) (width 0.4) (layer "F.Cu") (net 1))
 (segment (start 134.47 88.855) (end 134.47 89.505) (width 0.4) (layer "F.Cu") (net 1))
 (segment (start 130.48 89.04) (end 130.48 89.09) (width 0.4) (layer "F.Cu") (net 1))
 (segment (start 116.25 88.8) (end 114.59 87.14) (width 0.4) (layer "F.Cu") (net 1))
 (segment (start 138.445 84.955) (end 140.395 83.005) (width 0.4) (layer "F.Cu") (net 1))
 (segment (start 140.395 83.005) (end 141.77 83.005) (width 0.4) (layer "F.Cu") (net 1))
 (segment (start 145.9375 92.95) (end 145.9375 95.03) (width 0.4) (layer "F.Cu") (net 1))
 (segment (start 128.14 87.1875) (end 128.5775 87.1875) (width 0.4) (layer "F.Cu") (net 1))
 (segment (start 148.73 78.94) (end 149.63 79.84) (width 0.4) (layer "F.Cu") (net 1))
 (segment (start 137.795 85.605) (end 138.12 85.28) (width 0.4) (layer "F.Cu") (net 1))
 (segment (start 134.47 86.905) (end 136.495 86.905) (width 0.4) (layer "F.Cu") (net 1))
 (segment (start 145.8975 78.94) (end 148.73 78.94) (width 0.4) (layer "F.Cu") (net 1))
 (segment (start 125.2775 88.8) (end 116.25 88.8) (width 0.4) (layer "F.Cu") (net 1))
 (segment (start 145.9375 90.84) (end 145.9375 92.95) (width 0.4) (layer "F.Cu") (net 1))
 (segment (start 146.94 84.955) (end 156.695 84.955) (width 0.4) (layer "F.Cu") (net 1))
 (segment (start 156.7 86.8625) (end 156.69 86.8725) (width 0.4) (layer "F.Cu") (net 1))
 (segment (start 134.47 85.605) (end 137.795 85.605) (width 0.4) (layer "F.Cu") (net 1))
 (segment (start 145.8975 74.72) (end 145.8975 76.83) (width 0.5) (layer "F.Cu") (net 1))
 (segment (start 129.5125 82.49) (end 127.22 82.49) (width 0.4) (layer "F.Cu") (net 1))
 (segment (start 127.22 82.49) (end 126.89 82.49) (width 0.4) (layer "F.Cu") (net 1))
 (segment (start 145.8975 76.83) (end 145.8975 78.94) (width 0.4) (layer "F.Cu") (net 1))
 (segment (start 139.745 86.905) (end 138.12 85.28) (width 0.4) (layer "F.Cu") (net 1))
 (segment (start 156.7 84.96) (end 156.7 86.8625) (width 0.4) (layer "F.Cu") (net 1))
 (segment (start 156.7 83.0875) (end 156.7 84.96) (width 0.4) (layer "F.Cu") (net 1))
 (segment (start 114.59 87.14) (end 112.09 84.64) (width 0.4) (layer "F.Cu") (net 1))
 (segment (start 149.63 90.19) (end 149.63 85.81) (width 0.4) (layer "F.Cu") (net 1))
 (segment (start 141.77 86.905) (end 139.745 86.905) (width 0.4) (layer "F.Cu") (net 1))
 (segment (start 149.595 84.955) (end 146.94 84.955) (width 0.4) (layer "F.Cu") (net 1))
 (segment (start 145.9375 90.84) (end 148.98 90.84) (width 0.4) (layer "F.Cu") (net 1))
 (segment (start 126.89 87.1875) (end 128.14 87.1875) (width 0.4) (layer "F.Cu") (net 1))
 (segment (start 141.77 84.955) (end 138.445 84.955) (width 0.4) (layer "F.Cu") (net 1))
 (segment (start 126.89 82.49) (end 126.89 87.1875) (width 0.4) (layer "F.Cu") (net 1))
 (segment (start 149.63 85.81) (end 149.63 84.99) (width 0.4) (layer "F.Cu") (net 1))
 (segment (start 134.47 88.205) (end 134.47 88.855) (width 0.4) (layer "F.Cu") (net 1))
 (segment (start 127.22 82.49) (end 122.44 82.49) (width 0.4) (layer "F.Cu") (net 1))
 (segment (start 134.47 86.255) (end 134.47 86.905) (width 0.4) (layer "F.Cu") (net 1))
 (segment (start 135.195 88.205) (end 138.12 85.28) (width 0.4) (layer "F.Cu") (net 1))
 (segment (start 134.47 88.205) (end 135.195 88.205) (width 0.4) (layer "F.Cu") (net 1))
 (segment (start 122.44 82.49) (end 122.09 82.14) (width 0.4) (layer "F.Cu") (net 1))
 (segment (start 149.63 79.84) (end 149.63 85.81) (width 0.4) (layer "F.Cu") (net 1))
 (segment (start 132.615 86.905) (end 132.39 87.13) (width 0.4) (layer "F.Cu") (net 1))
 (segment (start 148.98 90.84) (end 149.63 90.19) (width 0.4) (layer "F.Cu") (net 1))
 (segment (start 112.09 84.64) (end 107.09 84.64) (width 0.4) (layer "F.Cu") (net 1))
 (segment (start 156.695 84.955) (end 156.7 84.96) (width 0.4) (layer "F.Cu") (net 1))
 (segment (start 141.77 84.955) (end 146.94 84.955) (width 0.4) (layer "F.Cu") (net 1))
 (segment (start 134.47 86.905) (end 132.615 86.905) (width 0.4) (layer "F.Cu") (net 1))
 (segment (start 126.89 87.1875) (end 125.2775 88.8) (width 0.4) (layer "F.Cu") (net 1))
 (segment (start 128.5775 87.1875) (end 130.48 89.09) (width 0.4) (layer "F.Cu") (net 1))
 (segment (start 149.63 84.99) (end 149.595 84.955) (width 0.4) (layer "F.Cu") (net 1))
 (segment (start 134.47 85.605) (end 134.47 86.255) (width 0.4) (layer "F.Cu") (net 1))
 (segment (start 132.39 87.13) (end 130.48 89.04) (width 0.4) (layer "F.Cu") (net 1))
 (segment (start 130.48 91.1725) (end 130.4725 91.18) (width 0.4) (layer "F.Cu") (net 1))
 (segment (start 133.735 87.555) (end 132.48 88.81) (width 0.4) (layer "F.Cu") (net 19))
 (segment (start 132.48 88.81) (end 132.48 89.09) (width 0.4) (layer "F.Cu") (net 19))
 (segment (start 134.47 87.555) (end 133.735 87.555) (width 0.4) (layer "F.Cu") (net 19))
 (segment (start 134.47 90.155) (end 133.5725 90.155) (width 0.4) (layer "F.Cu") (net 20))
 (segment (start 133.5725 90.155) (end 132.5475 91.18) (width 0.4) (layer "F.Cu") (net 20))
 (segment (start 143.8625 90.84) (end 143.8625 92.95) (width 0.4) (layer "F.Cu") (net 2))
 (segment (start 146.62 96.53) (end 152.25 90.9) (width 0.4) (layer "F.Cu") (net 2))
 (segment (start 162.46 79.1) (end 152.35 79.1) (width 0.4) (layer "F.Cu") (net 2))
 (segment (start 141.77 89.505) (end 141.77 90.155) (width 0.4) (layer "F.Cu") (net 2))
 (segment (start 145.13 96.53) (end 146.62 96.53) (width 0.4) (layer "F.Cu") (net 2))
 (segment (start 152.35 79.1) (end 146.56 73.31) (width 0.4) (layer "F.Cu") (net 2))
 (segment (start 143.8225 74.6975) (end 143.8225 74.72) (width 0.4) (layer "F.Cu") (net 2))
 (segment (start 164.94 81.58) (end 162.46 79.1) (width 0.4) (layer "F.Cu") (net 2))
 (segment (start 143.8625 92.95) (end 143.8625 95.03) (width 0.4) (layer "F.Cu") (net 2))
 (segment (start 142.3575 80.405) (end 143.8225 78.94) (width 0.4) (layer "F.Cu") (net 2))
 (segment (start 143.8725 95.04) (end 143.8725 95.2725) (width 0.4) (layer "F.Cu") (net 2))
 (segment (start 164.94 88.13) (end 164.94 81.58) (width 0.4) (layer "F.Cu") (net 2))
 (segment (start 152.25 90.9) (end 162.17 90.9) (width 0.4) (layer "F.Cu") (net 2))
 (segment (start 143.8725 95.2725) (end 145.13 96.53) (width 0.4) (layer "F.Cu") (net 2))
 (segment (start 141.77 80.405) (end 142.3575 80.405) (width 0.4) (layer "F.Cu") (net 2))
 (segment (start 146.56 73.31) (end 145.21 73.31) (width 0.4) (layer "F.Cu") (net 2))
 (segment (start 143.8225 76.83) (end 143.8225 78.94) (width 0.4) (layer "F.Cu") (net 2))
 (segment (start 141.77 90.155) (end 143.1775 90.155) (width 0.4) (layer "F.Cu") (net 2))
 (segment (start 143.8625 95.03) (end 143.8725 95.04) (width 0.4) (layer "F.Cu") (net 2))
 (segment (start 145.21 73.31) (end 143.8225 74.6975) (width 0.4) (layer "F.Cu") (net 2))
 (segment (start 141.77 88.855) (end 141.77 89.505) (width 0.4) (layer "F.Cu") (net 2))
 (segment (start 162.17 90.9) (end 164.94 88.13) (width 0.4) (layer "F.Cu") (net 2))
 (segment (start 141.77 80.405) (end 141.77 81.055) (width 0.4) (layer "F.Cu") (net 2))
 (segment (start 143.1775 90.155) (end 143.8625 90.84) (width 0.4) (layer "F.Cu") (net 2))
 (segment (start 143.8225 74.72) (end 143.8225 76.83) (width 0.5) (layer "F.Cu") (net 2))
 (segment (start 143.3375 88.205) (end 143.8425 88.71) (width 0.4) (layer "F.Cu") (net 14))
 (segment (start 141.77 88.205) (end 143.3375 88.205) (width 0.4) (layer "F.Cu") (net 14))
 (segment (start 145.9175 88.71) (end 145.9175 87.5625) (width 0.4) (layer "F.Cu") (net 11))
 (segment (start 145.9175 88.71) (end 147.82 88.71) (width 0.4) (layer "F.Cu") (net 11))
 (segment (start 142.47 87.555) (end 145.9 87.555) (width 0.4) (layer "F.Cu") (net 11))
 (segment (start 142.785 87.555) (end 142.8 87.54) (width 0.4) (layer "F.Cu") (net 11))
 (segment (start 145.9 87.555) (end 145.9175 87.5375) (width 0.4) (layer "F.Cu") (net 11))
 (segment (start 145.9175 86.4) (end 145.9175 87.5375) (width 0.4) (layer "F.Cu") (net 11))
 (segment (start 142.8 86.53) (end 142.525 86.255) (width 0.4) (layer "F.Cu") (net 11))
 (segment (start 147.82 88.71) (end 148.06 88.95) (width 0.4) (layer "F.Cu") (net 11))
 (segment (start 142.8 87.54) (end 142.8 86.53) (width 0.4) (layer "F.Cu") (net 11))
 (segment (start 141.77 87.555) (end 142.47 87.555) (width 0.4) (layer "F.Cu") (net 11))
 (segment (start 142.525 86.255) (end 141.77 86.255) (width 0.4) (layer "F.Cu") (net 11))
 (segment (start 142.47 87.555) (end 142.785 87.555) (width 0.4) (layer "F.Cu") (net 11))
 (segment (start 143.0475 85.605) (end 143.8425 86.4) (width 0.4) (layer "F.Cu") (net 10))
 (segment (start 141.77 85.605) (end 143.0475 85.605) (width 0.4) (layer "F.Cu") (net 10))
 (segment (start 143.0375 84.305) (end 143.8225 83.52) (width 0.4) (layer "F.Cu") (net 5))
 (segment (start 141.77 84.305) (end 143.0375 84.305) (width 0.4) (layer "F.Cu") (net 5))
 (segment (start 141.77 82.355) (end 142.5 82.355) (width 0.4) (layer "F.Cu") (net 6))
 (segment (start 142.5 82.355) (end 145.8725 82.355) (width 0.4) (layer "F.Cu") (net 6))
 (segment (start 142.795 82.355) (end 142.79 82.36) (width 0.4) (layer "F.Cu") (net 6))
 (segment (start 145.8975 81.2) (end 147.88 81.2) (width 0.4) (layer "F.Cu") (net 6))
 (segment (start 142.79 82.36) (end 142.79 83.37) (width 0.4) (layer "F.Cu") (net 6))
 (segment (start 142.5 82.355) (end 142.795 82.355) (width 0.4) (layer "F.Cu") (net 6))
 (segment (start 142.505 83.655) (end 141.77 83.655) (width 0.4) (layer "F.Cu") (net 6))
 (segment (start 147.88 81.2) (end 148.08 81) (width 0.4) (layer "F.Cu") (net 6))
 (segment (start 142.79 83.37) (end 142.505 83.655) (width 0.4) (layer "F.Cu") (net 6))
 (segment (start 145.8975 83.52) (end 145.8975 82.33) (width 0.4) (layer "F.Cu") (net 6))
 (segment (start 145.8725 82.355) (end 145.8975 82.33) (width 0.4) (layer "F.Cu") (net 6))
 (segment (start 145.8975 82.33) (end 145.8975 81.2) (width 0.4) (layer "F.Cu") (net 6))
 (segment (start 143.3175 81.705) (end 143.8225 81.2) (width 0.4) (layer "F.Cu") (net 12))
 (segment (start 141.77 81.705) (end 143.3175 81.705) (width 0.4) (layer "F.Cu") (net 12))
 (segment (start 154.4925 81.0125) (end 154.48 81) (width 0.4) (layer "F.Cu") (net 9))
 (segment (start 156.7 81.0125) (end 161.6925 81.0125) (width 0.4) (layer "F.Cu") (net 9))
 (segment (start 156.7 81.0125) (end 154.4925 81.0125) (width 0.4) (layer "F.Cu") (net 9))
 (segment (start 161.6925 81.0125) (end 163.02 82.34) (width 0.4) (layer "F.Cu") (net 9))
 (segment (start 154.46 88.95) (end 156.6875 88.95) (width 0.4) (layer "F.Cu") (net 13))
 (segment (start 156.69 88.9475) (end 161.4125 88.9475) (width 0.4) (layer "F.Cu") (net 13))
 (segment (start 161.4125 88.9475) (end 163.02 87.34) (width 0.4) (layer "F.Cu") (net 13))
 (segment (start 156.6875 88.95) (end 156.69 88.9475) (width 0.4) (layer "F.Cu") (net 13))
 (segment (start 120.55 80.42) (end 129.5125 80.42) (width 0.5) (layer "F.Cu") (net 8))
 (segment (start 119.47 84.52) (end 119.47 81.5) (width 0.5) (layer "F.Cu") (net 8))
 (segment (start 122.09 87.14) (end 119.47 84.52) (width 0.5) (layer "F.Cu") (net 8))
 (segment (start 119.47 81.5) (end 120.55 80.42) (width 0.5) (layer "F.Cu") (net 8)))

